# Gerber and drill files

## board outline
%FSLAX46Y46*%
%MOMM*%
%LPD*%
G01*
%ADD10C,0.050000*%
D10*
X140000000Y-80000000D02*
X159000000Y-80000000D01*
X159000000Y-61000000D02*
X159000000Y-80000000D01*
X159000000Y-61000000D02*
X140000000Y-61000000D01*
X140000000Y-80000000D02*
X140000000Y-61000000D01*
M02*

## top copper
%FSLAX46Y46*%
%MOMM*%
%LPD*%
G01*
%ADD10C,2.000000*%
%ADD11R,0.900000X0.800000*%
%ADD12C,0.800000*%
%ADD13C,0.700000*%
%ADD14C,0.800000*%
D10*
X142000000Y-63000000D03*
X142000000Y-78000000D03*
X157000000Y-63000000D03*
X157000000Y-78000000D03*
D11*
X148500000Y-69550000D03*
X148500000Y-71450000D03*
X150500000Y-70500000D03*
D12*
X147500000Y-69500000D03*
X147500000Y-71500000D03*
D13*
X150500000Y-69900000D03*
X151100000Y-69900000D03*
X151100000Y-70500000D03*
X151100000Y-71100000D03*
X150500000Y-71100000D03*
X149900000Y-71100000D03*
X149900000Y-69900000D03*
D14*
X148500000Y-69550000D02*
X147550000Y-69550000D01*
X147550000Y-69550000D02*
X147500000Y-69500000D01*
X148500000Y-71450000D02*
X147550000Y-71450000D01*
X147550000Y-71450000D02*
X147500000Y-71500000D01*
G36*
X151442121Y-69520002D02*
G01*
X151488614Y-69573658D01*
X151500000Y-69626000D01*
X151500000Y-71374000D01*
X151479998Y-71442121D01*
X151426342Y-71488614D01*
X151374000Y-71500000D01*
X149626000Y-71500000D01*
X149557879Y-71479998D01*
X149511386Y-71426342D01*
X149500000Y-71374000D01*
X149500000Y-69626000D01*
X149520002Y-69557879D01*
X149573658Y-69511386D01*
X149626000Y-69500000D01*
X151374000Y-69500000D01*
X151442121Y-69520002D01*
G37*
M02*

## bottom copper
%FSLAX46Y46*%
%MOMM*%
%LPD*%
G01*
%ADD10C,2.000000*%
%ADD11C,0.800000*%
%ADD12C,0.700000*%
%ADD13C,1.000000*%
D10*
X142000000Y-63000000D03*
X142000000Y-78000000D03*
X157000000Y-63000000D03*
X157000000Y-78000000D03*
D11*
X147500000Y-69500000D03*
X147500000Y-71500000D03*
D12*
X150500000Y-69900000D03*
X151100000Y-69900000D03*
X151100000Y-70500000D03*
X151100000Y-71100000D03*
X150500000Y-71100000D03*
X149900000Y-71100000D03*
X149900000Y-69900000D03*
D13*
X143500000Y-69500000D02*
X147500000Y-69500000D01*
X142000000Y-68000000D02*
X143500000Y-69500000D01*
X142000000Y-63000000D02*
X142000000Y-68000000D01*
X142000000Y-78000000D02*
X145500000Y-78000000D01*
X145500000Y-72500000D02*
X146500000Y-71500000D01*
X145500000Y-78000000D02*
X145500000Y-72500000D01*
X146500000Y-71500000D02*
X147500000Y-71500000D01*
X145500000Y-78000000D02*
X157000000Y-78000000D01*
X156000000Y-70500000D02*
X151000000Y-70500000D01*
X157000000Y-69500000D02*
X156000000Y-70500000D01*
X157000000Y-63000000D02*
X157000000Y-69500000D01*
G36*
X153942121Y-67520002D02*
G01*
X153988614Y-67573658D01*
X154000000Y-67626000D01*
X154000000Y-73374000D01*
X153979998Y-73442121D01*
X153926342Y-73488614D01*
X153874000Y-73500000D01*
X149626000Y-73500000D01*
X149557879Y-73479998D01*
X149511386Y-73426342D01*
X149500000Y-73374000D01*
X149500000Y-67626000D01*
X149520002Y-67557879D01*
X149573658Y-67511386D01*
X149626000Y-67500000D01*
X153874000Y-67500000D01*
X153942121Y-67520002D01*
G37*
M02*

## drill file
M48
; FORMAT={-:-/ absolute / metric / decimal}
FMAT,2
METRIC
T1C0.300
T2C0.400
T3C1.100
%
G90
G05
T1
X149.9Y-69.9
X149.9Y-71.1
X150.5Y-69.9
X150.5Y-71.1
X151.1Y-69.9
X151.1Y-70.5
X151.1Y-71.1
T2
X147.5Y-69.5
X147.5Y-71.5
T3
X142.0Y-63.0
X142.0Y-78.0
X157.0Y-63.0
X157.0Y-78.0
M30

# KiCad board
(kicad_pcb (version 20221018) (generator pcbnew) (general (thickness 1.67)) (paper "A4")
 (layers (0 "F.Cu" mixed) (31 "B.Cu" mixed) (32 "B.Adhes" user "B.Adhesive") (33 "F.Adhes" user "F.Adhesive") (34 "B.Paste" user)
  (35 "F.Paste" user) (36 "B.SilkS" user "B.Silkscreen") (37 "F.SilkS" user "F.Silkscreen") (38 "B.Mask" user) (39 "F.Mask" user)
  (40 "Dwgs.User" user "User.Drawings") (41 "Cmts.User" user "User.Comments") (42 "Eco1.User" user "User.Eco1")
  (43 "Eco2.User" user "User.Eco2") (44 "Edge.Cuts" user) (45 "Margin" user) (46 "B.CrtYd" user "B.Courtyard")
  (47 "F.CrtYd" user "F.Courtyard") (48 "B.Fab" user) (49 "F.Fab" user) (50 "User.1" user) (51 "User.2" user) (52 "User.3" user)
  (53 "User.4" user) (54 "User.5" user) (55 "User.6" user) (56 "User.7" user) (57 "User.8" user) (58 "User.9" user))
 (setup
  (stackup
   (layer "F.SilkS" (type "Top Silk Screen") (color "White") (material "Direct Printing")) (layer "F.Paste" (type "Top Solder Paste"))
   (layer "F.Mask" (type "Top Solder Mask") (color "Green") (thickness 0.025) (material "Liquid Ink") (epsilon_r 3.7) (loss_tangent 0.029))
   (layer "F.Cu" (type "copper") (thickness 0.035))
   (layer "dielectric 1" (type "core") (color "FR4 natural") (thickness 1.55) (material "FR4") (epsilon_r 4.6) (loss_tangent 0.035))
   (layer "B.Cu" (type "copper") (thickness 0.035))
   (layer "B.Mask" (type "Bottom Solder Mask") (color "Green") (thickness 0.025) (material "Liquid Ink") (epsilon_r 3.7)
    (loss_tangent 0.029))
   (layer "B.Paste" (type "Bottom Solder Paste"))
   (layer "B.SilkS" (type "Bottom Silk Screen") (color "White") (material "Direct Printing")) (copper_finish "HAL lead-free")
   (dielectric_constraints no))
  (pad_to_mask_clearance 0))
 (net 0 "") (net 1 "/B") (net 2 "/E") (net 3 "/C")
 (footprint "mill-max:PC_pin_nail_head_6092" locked (layer "F.Cu") (at 142 63)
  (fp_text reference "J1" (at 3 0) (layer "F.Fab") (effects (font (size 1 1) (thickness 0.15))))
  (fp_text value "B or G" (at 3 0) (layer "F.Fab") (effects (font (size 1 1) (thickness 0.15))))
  (pad "1" thru_hole circle locked (at 0 0) (size 2 2) (drill 1.1) (layers "*.Cu" "*.Mask") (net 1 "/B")))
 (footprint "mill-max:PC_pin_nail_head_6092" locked (layer "F.Cu") (at 142 78)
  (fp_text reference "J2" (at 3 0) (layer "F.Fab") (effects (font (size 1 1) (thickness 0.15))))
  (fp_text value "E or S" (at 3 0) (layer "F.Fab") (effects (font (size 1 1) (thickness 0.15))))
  (pad "1" thru_hole circle locked (at 0 0) (size 2 2) (drill 1.1) (layers "*.Cu" "*.Mask") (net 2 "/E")))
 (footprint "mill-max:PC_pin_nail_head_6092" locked (layer "F.Cu") (at 157 63)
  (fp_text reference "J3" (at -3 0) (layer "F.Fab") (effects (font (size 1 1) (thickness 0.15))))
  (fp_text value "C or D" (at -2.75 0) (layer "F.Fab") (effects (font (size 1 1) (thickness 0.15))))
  (pad "1" thru_hole circle locked (at 0 0) (size 2 2) (drill 1.1) (layers "*.Cu" "*.Mask") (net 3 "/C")))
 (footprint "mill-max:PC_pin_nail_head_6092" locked (layer "F.Cu") (at 157 78)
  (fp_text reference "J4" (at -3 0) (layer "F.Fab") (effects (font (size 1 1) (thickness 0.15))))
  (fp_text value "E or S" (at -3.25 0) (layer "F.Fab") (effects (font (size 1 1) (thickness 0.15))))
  (pad "1" thru_hole circle locked (at 0 0) (size 2 2) (drill 1.1) (layers "*.Cu" "*.Mask") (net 2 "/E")))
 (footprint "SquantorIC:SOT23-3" (layer "F.Cu") (at 149.5 70.5)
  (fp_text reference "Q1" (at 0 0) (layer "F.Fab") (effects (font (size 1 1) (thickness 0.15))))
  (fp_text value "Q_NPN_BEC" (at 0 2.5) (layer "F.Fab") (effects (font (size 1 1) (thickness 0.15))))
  (pad "1" smd rect (at -1 -0.95 270) (size 0.8 0.9) (layers "F.Cu" "F.Paste" "F.Mask") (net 1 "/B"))
  (pad "2" smd rect (at -1 0.95 270) (size 0.8 0.9) (layers "F.Cu" "F.Paste" "F.Mask") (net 2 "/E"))
  (pad "3" smd rect (at 1 0 270) (size 0.8 0.9) (layers "F.Cu" "F.Paste" "F.Mask") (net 3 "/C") (zone_connect 2)))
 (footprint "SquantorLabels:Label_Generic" (layer "B.Cu") (at 157.25 71.5 90)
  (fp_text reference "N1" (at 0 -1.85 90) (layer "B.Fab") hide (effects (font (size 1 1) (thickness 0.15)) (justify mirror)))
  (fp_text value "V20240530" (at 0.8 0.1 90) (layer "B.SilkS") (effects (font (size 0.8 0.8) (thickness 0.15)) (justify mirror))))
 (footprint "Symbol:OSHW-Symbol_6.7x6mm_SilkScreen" (layer "B.Cu") (at 153.75 70.5 -90)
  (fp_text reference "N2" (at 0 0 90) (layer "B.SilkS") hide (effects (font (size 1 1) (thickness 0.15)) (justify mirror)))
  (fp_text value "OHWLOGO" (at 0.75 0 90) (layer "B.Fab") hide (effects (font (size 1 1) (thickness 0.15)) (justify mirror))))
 (gr_line (start 140 80) (end 159 80) (stroke (width 0.05) (type solid)) (layer "Edge.Cuts"))
 (gr_line (start 159 61) (end 159 80) (stroke (width 0.05) (type solid)) (layer "Edge.Cuts"))
 (gr_line (start 159 61) (end 140 61) (stroke (width 0.05) (type solid)) (layer "Edge.Cuts"))
 (gr_line (start 140 80) (end 140 61) (stroke (width 0.05) (type solid)) (layer "Edge.Cuts"))
 (segment (start 148.5 69.55) (end 147.55 69.55) (width 0.8) (layer "F.Cu") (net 1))
 (segment (start 147.55 69.55) (end 147.5 69.5) (width 0.8) (layer "F.Cu") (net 1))
 (via (at 147.5 69.5) (size 0.8) (drill 0.4) (layers "F.Cu" "B.Cu") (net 1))
 (segment (start 143.5 69.5) (end 147.5 69.5) (width 1) (layer "B.Cu") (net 1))
 (segment (start 142 68) (end 143.5 69.5) (width 1) (layer "B.Cu") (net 1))
 (segment (start 142 63) (end 142 68) (width 1) (layer "B.Cu") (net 1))
 (segment (start 148.5 71.45) (end 147.55 71.45) (width 0.8) (layer "F.Cu") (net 2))
 (segment (start 147.55 71.45) (end 147.5 71.5) (width 0.8) (layer "F.Cu") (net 2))
 (via (at 147.5 71.5) (size 0.8) (drill 0.4) (layers "F.Cu" "B.Cu") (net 2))
 (segment (start 142 78) (end 145.5 78) (width 1) (layer "B.Cu") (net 2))
 (segment (start 145.5 72.5) (end 146.5 71.5) (width 1) (layer "B.Cu") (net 2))
 (segment (start 145.5 78) (end 145.5 72.5) (width 1) (layer "B.Cu") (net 2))
 (segment (start 146.5 71.5) (end 147.5 71.5) (width 1) (layer "B.Cu") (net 2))
 (segment (start 145.5 78) (end 157 78) (width 1) (layer "B.Cu") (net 2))
 (via (at 150.5 69.9) (size 0.7) (drill 0.3) (layers "F.Cu" "B.Cu") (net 3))
 (via (at 151.1 69.9) (size 0.7) (drill 0.3) (layers "F.Cu" "B.Cu") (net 3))
 (via (at 151.1 70.5) (size 0.7) (drill 0.3) (layers "F.Cu" "B.Cu") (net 3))
 (via (at 151.1 71.1) (size 0.7) (drill 0.3) (layers "F.Cu" "B.Cu") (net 3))
 (via (at 150.5 71.1) (size 0.7) (drill 0.3) (layers "F.Cu" "B.Cu") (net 3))
 (via (at 149.9 71.1) (size 0.7) (drill 0.3) (layers "F.Cu" "B.Cu") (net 3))
 (via (at 149.9 69.9) (size 0.7) (drill 0.3) (layers "F.Cu" "B.Cu") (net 3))
 (segment (start 156 70.5) (end 151 70.5) (width 1) (layer "B.Cu") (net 3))
 (segment (start 157 69.5) (end 156 70.5) (width 1) (layer "B.Cu") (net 3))
 (segment (start 157 63) (end 157 69.5) (width 1) (layer "B.Cu") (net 3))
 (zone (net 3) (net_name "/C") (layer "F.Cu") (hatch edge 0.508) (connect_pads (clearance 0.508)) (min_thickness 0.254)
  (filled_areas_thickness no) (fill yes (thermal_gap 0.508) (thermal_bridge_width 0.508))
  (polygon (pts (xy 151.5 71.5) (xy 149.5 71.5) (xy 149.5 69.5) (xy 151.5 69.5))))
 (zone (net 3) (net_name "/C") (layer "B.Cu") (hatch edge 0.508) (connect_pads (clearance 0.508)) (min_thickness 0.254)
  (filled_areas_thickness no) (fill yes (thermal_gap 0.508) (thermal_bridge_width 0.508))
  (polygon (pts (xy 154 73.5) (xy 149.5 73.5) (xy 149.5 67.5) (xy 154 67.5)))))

